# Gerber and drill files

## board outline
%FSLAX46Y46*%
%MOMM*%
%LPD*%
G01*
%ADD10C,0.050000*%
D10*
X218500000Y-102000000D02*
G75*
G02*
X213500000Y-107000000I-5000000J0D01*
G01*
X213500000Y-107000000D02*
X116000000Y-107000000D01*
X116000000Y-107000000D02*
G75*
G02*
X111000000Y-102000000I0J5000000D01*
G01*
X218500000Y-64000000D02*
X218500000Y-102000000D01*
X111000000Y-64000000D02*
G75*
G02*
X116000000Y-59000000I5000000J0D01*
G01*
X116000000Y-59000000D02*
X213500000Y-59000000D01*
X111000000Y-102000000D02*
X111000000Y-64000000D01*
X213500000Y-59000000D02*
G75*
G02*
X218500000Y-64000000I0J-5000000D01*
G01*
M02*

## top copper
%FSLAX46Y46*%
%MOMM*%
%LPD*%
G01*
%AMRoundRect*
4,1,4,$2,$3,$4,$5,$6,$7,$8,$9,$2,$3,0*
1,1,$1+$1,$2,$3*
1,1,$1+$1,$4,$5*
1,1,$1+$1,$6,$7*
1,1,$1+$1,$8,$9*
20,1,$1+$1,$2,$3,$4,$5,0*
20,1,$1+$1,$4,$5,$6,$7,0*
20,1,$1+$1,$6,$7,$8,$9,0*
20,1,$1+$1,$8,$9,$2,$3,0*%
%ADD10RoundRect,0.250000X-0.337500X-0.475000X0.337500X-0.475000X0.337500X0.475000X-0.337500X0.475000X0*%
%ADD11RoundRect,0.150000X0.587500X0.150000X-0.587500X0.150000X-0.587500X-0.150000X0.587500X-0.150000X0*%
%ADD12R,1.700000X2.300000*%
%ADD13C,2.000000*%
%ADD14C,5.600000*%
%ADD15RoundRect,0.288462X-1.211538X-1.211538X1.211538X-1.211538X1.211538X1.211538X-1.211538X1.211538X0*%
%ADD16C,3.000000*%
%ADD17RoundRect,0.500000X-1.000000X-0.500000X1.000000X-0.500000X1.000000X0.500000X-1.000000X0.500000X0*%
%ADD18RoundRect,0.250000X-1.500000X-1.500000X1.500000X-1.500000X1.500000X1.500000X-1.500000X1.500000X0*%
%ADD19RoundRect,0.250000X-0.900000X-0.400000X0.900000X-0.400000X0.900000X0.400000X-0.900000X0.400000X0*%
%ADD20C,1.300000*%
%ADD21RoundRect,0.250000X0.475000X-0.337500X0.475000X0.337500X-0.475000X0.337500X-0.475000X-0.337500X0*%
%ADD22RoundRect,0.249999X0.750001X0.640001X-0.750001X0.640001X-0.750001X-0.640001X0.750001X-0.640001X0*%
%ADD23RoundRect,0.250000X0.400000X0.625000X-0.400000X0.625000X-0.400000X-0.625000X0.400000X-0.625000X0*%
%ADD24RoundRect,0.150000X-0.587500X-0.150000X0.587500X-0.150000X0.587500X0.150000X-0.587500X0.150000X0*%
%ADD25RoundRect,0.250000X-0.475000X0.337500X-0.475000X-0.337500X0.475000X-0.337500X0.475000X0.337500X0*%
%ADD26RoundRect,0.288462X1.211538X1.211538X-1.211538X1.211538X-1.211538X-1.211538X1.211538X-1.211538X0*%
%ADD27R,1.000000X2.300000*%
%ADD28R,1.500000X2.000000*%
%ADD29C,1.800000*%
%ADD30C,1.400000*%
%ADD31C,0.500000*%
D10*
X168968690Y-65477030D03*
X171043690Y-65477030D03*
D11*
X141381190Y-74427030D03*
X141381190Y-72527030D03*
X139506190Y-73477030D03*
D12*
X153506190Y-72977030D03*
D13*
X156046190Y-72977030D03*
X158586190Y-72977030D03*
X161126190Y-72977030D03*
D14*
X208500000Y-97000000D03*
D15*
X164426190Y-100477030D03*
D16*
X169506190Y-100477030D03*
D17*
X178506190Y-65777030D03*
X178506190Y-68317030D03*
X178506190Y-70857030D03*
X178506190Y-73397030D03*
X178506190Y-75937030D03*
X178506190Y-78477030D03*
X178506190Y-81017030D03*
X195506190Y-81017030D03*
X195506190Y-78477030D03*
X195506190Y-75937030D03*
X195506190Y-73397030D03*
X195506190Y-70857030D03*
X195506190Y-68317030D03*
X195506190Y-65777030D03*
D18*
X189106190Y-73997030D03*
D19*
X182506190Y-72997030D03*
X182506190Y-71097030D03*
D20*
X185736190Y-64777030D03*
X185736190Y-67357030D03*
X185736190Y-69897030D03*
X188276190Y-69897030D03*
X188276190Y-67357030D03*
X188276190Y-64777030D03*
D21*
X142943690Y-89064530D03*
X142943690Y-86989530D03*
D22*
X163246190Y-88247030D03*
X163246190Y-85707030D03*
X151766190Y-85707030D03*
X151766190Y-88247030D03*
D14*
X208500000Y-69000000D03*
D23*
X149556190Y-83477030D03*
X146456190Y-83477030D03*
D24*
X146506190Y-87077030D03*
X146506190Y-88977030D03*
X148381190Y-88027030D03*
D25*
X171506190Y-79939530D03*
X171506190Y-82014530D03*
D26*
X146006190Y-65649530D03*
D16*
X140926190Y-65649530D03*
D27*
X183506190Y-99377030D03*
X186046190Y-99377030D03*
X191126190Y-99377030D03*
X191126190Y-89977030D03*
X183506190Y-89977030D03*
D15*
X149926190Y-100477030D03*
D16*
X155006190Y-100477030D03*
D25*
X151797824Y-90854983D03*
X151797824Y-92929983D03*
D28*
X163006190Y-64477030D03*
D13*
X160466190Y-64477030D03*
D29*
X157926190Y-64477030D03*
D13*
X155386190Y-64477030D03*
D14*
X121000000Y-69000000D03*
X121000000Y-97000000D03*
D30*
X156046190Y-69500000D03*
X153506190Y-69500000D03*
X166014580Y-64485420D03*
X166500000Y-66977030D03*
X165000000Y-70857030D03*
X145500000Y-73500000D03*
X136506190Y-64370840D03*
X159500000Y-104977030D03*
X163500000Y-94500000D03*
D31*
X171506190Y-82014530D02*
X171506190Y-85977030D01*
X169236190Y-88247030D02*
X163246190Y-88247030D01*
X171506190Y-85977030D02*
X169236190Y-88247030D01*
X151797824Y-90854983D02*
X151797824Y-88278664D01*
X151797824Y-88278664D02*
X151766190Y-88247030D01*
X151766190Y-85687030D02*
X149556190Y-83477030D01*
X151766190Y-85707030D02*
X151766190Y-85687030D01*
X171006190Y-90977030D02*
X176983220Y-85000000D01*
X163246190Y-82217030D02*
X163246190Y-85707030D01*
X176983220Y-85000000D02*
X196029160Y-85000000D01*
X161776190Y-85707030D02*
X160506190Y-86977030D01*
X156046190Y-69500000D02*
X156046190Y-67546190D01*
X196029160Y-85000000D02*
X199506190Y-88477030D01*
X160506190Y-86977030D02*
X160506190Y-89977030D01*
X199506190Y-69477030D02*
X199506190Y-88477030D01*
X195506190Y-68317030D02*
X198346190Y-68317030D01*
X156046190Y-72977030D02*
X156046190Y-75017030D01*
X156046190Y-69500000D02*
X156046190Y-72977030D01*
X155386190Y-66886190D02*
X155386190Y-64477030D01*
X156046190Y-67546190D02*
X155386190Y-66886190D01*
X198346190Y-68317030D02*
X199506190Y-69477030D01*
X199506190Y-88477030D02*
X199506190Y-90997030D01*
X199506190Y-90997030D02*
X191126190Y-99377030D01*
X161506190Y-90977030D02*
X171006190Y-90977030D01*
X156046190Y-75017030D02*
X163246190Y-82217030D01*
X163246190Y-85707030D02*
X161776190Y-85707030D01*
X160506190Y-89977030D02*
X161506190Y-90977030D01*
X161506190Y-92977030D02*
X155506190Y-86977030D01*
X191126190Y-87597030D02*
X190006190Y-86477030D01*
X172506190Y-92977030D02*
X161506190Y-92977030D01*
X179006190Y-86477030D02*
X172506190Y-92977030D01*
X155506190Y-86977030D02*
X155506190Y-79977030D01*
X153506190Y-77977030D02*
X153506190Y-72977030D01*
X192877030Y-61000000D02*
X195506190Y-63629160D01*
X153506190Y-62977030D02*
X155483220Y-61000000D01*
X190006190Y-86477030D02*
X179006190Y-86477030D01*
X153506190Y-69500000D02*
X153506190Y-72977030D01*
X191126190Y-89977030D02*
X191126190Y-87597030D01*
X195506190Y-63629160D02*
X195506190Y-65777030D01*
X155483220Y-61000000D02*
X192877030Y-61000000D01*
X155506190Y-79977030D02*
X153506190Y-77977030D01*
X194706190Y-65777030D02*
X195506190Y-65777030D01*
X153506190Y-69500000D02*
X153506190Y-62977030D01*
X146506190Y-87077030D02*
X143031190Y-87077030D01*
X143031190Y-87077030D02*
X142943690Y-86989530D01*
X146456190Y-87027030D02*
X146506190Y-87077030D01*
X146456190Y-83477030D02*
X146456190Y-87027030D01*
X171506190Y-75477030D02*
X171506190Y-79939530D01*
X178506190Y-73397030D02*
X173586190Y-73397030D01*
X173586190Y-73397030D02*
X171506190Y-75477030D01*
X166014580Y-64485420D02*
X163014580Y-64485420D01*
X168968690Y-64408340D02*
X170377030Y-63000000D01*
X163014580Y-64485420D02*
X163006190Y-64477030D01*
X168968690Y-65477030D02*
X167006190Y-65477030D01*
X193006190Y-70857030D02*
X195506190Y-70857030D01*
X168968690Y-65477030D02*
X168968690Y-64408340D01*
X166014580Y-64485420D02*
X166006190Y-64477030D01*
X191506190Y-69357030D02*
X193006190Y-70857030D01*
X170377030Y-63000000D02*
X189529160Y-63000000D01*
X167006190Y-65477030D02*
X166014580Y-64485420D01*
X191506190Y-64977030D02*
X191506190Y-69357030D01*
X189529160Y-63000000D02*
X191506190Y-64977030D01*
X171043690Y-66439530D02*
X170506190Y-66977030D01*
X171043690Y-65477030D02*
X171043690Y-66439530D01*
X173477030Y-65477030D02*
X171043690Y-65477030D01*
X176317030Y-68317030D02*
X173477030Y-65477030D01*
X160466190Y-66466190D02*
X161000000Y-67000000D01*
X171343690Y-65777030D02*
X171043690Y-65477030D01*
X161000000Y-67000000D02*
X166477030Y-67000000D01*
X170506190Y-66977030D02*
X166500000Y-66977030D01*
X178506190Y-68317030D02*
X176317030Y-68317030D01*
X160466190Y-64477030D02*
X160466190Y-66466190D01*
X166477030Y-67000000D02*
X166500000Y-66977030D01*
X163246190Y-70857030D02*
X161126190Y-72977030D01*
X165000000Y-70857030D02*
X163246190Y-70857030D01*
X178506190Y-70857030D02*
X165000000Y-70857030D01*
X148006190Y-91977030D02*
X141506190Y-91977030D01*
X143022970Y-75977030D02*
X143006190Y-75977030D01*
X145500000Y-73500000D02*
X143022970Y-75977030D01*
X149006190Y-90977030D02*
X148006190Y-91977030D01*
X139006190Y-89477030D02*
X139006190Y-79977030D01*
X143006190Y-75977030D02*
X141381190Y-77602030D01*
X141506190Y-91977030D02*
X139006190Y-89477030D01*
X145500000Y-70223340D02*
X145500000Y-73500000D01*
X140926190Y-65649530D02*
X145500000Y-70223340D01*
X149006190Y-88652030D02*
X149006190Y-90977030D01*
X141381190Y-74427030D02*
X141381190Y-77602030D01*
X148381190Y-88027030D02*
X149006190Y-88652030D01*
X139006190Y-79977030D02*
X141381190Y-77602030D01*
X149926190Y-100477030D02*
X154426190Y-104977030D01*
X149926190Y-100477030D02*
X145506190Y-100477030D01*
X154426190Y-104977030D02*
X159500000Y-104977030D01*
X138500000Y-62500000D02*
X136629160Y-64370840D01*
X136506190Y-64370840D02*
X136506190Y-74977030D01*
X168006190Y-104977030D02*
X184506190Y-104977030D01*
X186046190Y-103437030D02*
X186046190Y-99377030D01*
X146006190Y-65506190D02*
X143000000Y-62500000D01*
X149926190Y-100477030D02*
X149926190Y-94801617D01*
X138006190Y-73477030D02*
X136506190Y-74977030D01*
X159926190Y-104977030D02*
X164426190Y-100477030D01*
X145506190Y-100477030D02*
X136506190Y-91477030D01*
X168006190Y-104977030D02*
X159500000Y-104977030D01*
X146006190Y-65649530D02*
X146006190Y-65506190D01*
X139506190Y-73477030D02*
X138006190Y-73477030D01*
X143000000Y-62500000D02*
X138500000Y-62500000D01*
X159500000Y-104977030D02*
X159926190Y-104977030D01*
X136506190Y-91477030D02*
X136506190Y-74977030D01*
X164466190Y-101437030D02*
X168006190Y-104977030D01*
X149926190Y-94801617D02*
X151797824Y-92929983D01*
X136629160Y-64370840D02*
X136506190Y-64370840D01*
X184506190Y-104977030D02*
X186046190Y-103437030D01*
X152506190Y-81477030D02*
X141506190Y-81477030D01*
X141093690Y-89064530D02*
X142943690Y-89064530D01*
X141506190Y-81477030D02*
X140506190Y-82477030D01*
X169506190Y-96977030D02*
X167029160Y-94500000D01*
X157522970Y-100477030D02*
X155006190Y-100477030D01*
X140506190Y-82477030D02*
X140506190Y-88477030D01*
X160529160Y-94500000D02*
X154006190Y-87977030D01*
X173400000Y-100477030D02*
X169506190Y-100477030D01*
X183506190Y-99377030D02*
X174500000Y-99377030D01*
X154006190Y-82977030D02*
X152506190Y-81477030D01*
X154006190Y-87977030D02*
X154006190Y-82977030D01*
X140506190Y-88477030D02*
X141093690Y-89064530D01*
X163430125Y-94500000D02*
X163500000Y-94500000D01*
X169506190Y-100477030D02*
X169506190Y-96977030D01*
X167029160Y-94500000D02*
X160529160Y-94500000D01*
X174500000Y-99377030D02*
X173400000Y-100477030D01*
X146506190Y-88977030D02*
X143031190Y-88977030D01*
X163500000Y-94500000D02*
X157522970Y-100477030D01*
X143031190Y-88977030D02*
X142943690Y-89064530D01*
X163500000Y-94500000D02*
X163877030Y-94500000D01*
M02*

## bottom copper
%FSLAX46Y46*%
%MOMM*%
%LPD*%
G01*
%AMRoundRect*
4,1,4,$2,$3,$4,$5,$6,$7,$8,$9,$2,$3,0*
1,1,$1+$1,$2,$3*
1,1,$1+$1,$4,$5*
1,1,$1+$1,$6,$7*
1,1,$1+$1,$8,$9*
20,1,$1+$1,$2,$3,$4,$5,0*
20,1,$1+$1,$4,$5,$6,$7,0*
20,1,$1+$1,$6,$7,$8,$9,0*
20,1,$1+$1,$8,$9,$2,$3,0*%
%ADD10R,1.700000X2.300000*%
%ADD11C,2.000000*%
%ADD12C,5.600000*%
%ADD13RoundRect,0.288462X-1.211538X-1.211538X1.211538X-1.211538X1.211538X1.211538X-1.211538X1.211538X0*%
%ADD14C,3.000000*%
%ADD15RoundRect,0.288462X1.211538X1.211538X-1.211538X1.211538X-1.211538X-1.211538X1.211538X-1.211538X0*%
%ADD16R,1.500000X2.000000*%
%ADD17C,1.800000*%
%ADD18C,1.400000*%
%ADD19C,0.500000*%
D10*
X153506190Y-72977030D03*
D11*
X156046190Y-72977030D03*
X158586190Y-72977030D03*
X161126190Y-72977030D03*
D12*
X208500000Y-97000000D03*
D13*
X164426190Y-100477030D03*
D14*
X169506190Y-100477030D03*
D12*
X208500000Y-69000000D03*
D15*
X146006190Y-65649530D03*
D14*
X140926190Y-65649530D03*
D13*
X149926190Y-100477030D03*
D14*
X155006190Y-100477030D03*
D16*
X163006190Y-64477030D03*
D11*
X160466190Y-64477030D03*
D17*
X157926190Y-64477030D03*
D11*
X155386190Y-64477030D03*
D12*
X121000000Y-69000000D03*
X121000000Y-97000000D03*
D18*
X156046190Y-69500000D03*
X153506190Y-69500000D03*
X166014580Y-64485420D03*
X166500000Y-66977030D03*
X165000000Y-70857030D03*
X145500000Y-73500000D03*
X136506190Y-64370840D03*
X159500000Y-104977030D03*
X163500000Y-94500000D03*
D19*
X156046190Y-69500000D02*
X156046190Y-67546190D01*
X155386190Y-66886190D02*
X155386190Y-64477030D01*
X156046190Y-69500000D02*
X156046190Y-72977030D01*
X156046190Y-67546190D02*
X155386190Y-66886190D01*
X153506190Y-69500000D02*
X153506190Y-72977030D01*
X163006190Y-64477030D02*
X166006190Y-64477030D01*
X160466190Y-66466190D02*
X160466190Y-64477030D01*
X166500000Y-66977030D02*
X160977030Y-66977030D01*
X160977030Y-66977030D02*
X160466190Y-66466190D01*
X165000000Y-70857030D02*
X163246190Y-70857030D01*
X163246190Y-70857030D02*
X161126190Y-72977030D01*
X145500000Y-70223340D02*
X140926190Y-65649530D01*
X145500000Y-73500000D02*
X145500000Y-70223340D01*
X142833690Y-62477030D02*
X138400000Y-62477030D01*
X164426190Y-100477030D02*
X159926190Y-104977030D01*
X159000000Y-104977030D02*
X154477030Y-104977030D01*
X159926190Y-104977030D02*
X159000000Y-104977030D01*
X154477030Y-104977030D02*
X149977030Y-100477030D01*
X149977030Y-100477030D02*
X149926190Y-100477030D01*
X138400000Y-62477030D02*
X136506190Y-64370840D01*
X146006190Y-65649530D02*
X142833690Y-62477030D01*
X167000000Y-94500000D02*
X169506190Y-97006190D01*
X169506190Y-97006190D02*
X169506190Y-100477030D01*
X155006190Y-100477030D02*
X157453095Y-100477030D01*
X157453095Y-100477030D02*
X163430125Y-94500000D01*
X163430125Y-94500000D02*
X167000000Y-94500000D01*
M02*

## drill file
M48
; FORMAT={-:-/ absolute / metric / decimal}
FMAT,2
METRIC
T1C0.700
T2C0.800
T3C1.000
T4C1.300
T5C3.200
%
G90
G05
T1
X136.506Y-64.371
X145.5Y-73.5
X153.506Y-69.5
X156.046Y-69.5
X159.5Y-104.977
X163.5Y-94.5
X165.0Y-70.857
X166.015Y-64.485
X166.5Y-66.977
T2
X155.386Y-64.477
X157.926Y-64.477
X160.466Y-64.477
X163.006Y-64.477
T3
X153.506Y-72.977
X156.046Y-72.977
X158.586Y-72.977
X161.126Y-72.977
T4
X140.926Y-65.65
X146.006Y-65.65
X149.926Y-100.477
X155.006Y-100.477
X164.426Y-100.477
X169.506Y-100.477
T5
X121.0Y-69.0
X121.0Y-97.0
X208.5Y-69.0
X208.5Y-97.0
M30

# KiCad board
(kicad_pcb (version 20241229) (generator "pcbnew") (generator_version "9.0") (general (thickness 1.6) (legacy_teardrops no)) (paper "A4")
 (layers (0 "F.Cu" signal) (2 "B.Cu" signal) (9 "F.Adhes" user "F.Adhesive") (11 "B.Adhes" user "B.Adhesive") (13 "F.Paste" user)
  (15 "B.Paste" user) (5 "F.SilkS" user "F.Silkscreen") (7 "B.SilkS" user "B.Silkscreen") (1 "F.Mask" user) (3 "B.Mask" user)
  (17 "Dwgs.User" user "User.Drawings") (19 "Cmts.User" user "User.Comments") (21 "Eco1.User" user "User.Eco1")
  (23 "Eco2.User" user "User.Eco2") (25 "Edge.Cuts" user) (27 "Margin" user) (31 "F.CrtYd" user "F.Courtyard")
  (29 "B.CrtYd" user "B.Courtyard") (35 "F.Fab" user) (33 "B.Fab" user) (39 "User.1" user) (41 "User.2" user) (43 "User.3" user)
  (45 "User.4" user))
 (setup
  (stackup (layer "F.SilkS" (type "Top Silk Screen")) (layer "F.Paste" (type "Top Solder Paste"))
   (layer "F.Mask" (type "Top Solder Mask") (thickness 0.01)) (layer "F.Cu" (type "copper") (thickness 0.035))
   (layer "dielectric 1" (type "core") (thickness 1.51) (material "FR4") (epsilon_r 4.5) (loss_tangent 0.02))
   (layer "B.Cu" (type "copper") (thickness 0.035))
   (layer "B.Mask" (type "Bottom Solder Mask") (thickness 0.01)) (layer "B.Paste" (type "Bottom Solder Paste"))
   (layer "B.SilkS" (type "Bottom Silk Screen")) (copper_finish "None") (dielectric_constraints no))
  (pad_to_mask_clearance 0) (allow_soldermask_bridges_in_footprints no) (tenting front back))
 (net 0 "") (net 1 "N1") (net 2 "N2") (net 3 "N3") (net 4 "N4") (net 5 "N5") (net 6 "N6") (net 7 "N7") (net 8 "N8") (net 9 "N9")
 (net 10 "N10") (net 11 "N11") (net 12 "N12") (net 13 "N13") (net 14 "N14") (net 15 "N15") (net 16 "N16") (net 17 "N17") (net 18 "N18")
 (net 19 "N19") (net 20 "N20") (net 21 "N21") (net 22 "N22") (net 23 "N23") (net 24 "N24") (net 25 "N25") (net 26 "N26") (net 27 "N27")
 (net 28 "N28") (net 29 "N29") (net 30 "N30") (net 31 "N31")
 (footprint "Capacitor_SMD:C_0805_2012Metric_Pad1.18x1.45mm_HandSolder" (layer "F.Cu") (at 170.00619 65.47703)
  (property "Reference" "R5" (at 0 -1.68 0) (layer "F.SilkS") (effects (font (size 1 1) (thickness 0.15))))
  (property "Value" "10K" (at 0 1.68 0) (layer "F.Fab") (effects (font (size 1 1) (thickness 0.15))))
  (pad "1" smd roundrect (at -1.0375 0) (size 1.175 1.45) (layers "F.Cu" "F.Mask" "F.Paste") (roundrect_rratio 0.212766) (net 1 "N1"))
  (pad "2" smd roundrect (at 1.0375 0) (size 1.175 1.45) (layers "F.Cu" "F.Mask" "F.Paste") (roundrect_rratio 0.212766) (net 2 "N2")))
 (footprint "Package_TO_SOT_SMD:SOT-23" (layer "F.Cu") (at 140.44369 73.47703 180)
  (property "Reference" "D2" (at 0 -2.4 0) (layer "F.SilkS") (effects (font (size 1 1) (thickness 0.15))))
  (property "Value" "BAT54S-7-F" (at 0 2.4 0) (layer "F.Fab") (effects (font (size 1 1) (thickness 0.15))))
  (pad "1" smd roundrect (at -0.9375 -0.95 180) (size 1.475 0.6) (layers "F.Cu" "F.Mask" "F.Paste") (roundrect_rratio 0.25) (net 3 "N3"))
  (pad "2" smd roundrect (at -0.9375 0.95 180) (size 1.475 0.6) (layers "F.Cu" "F.Mask" "F.Paste") (roundrect_rratio 0.25) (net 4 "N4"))
  (pad "3" smd roundrect (at 0.9375 0 180) (size 1.475 0.6) (layers "F.Cu" "F.Mask" "F.Paste") (roundrect_rratio 0.25) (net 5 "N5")))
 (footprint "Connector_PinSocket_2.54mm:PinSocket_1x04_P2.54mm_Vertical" (layer "F.Cu") (at 153.50619 72.97703 90)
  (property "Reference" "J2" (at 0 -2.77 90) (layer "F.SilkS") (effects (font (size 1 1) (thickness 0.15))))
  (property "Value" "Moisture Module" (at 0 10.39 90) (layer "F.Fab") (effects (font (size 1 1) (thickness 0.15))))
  (pad "1" thru_hole rect (at 0 0 90) (size 2.3 1.7) (drill 1) (layers "*.Cu" "*.Mask") (remove_unused_layers no) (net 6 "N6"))
  (pad "2" thru_hole circle (at 0 2.54 90) (size 2 2) (drill 1) (layers "*.Cu" "*.Mask") (remove_unused_layers no) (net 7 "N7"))
  (pad "3" thru_hole circle (at 0 5.08 90) (size 2 2) (drill 1) (layers "*.Cu" "*.Mask") (remove_unused_layers no) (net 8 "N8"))
  (pad "4" thru_hole circle (at 0 7.62 90) (size 2 2) (drill 1) (layers "*.Cu" "*.Mask") (remove_unused_layers no) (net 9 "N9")))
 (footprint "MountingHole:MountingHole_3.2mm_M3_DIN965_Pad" (layer "F.Cu") (at 208.5 97)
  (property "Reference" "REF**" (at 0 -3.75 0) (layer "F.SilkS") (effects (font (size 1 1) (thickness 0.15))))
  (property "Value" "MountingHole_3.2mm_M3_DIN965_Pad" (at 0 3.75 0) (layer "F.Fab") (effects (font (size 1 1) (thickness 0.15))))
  (pad "1" thru_hole circle (at 0 0) (size 5.6 5.6) (drill 3.2) (layers "*.Cu" "*.Mask") (remove_unused_layers no) (zone_connect 2)))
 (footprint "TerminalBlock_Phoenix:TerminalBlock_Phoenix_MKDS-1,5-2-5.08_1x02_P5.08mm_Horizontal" (layer "F.Cu") (at 164.42619 100.47703)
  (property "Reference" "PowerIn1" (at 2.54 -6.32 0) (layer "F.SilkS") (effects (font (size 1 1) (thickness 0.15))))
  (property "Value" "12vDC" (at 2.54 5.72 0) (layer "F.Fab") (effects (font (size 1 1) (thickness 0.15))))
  (pad "1" thru_hole roundrect (at 0 0) (size 3 3) (drill 1.3) (layers "*.Cu" "*.Mask") (remove_unused_layers no)
   (roundrect_rratio 0.096154) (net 5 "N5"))
  (pad "2" thru_hole circle (at 5.08 0) (size 3 3) (drill 1.3) (layers "*.Cu" "*.Mask") (remove_unused_layers no) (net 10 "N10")))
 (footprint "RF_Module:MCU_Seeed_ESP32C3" (layer "F.Cu") (at 187.00619 73.39703)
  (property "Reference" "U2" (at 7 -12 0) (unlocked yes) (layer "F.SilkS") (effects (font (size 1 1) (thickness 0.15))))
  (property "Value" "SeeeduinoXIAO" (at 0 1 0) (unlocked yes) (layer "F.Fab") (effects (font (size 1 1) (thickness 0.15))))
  (pad "" smd roundrect (at 1.1 -0.4) (size 1.5 1.5) (layers "F.Paste") (roundrect_rratio 0.1666666667))
  (pad "" smd roundrect (at 1.1 1.6) (size 1.5 1.5) (layers "F.Paste") (roundrect_rratio 0.1666666667))
  (pad "" smd roundrect (at 3.1 -0.4) (size 1.5 1.5) (layers "F.Paste") (roundrect_rratio 0.1666666667))
  (pad "" smd roundrect (at 3.1 1.6) (size 1.5 1.5) (layers "F.Paste") (roundrect_rratio 0.1666666667))
  (pad "1" smd roundrect (at -8.5 -7.62) (size 3 2) (layers "F.Cu" "F.Mask" "F.Paste") (roundrect_rratio 0.25) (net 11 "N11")
   (thermal_bridge_angle 45))
  (pad "2" smd roundrect (at -8.5 -5.08) (size 3 2) (layers "F.Cu" "F.Mask" "F.Paste") (roundrect_rratio 0.25) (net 2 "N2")
   (thermal_bridge_angle 45))
  (pad "3" smd roundrect (at -8.5 -2.54) (size 3 2) (layers "F.Cu" "F.Mask" "F.Paste") (roundrect_rratio 0.25) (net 9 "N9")
   (thermal_bridge_angle 45))
  (pad "4" smd roundrect (at -8.5 0) (size 3 2) (layers "F.Cu" "F.Mask" "F.Paste") (roundrect_rratio 0.25) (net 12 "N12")
   (thermal_bridge_angle 45))
  (pad "5" smd roundrect (at -8.5 2.54) (size 3 2) (layers "F.Cu" "F.Mask" "F.Paste") (roundrect_rratio 0.25) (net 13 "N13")
   (thermal_bridge_angle 45))
  (pad "6" smd roundrect (at -8.5 5.08) (size 3 2) (layers "F.Cu" "F.Mask" "F.Paste") (roundrect_rratio 0.25) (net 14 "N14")
   (thermal_bridge_angle 45))
  (pad "7" smd roundrect (at -8.5 7.62) (size 3 2) (layers "F.Cu" "F.Mask" "F.Paste") (roundrect_rratio 0.25) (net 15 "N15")
   (thermal_bridge_angle 45))
  (pad "8" smd roundrect (at 8.5 7.62) (size 3 2) (layers "F.Cu" "F.Mask" "F.Paste") (roundrect_rratio 0.25) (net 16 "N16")
   (thermal_bridge_angle 45))
  (pad "9" smd roundrect (at 8.5 5.08) (size 3 2) (layers "F.Cu" "F.Mask" "F.Paste") (roundrect_rratio 0.25) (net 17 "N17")
   (thermal_bridge_angle 45))
  (pad "10" smd roundrect (at 8.5 2.54) (size 3 2) (layers "F.Cu" "F.Mask" "F.Paste") (roundrect_rratio 0.25) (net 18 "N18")
   (thermal_bridge_angle 45))
  (pad "11" smd roundrect (at 8.5 0) (size 3 2) (layers "F.Cu" "F.Mask" "F.Paste") (roundrect_rratio 0.25) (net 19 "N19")
   (thermal_bridge_angle 45))
  (pad "12" smd roundrect (at 8.5 -2.54) (size 3 2) (layers "F.Cu" "F.Mask" "F.Paste") (roundrect_rratio 0.25) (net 1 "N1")
   (thermal_bridge_angle 45))
  (pad "13" smd roundrect (at 8.5 -5.08) (size 3 2) (layers "F.Cu" "F.Mask" "F.Paste") (roundrect_rratio 0.25) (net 7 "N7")
   (thermal_bridge_angle 45))
  (pad "14" smd roundrect (at 8.5 -7.62) (size 3 2) (layers "F.Cu" "F.Mask" "F.Paste") (roundrect_rratio 0.25) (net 6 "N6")
   (thermal_bridge_angle 45))
  (pad "15" smd roundrect (at 2.1 0.6) (size 3.5 3.5) (layers "F.Cu" "F.Mask") (roundrect_rratio 0.07142857143) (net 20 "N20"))
  (pad "16" smd roundrect (at -4.5 -0.4) (size 2.3 1.3) (layers "F.Cu" "F.Mask" "F.Paste") (roundrect_rratio 0.1923076923) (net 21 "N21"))
  (pad "17" smd roundrect (at -4.5 -2.3) (size 2.3 1.3) (layers "F.Cu" "F.Mask" "F.Paste") (roundrect_rratio 0.1923076923) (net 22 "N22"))
  (pad "18" smd circle (at -1.27 -8.62) (size 1.3 1.3) (layers "F.Cu" "F.Mask" "F.Paste") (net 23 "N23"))
  (pad "19" smd circle (at -1.27 -6.04) (size 1.3 1.3) (layers "F.Cu" "F.Mask" "F.Paste") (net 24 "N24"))
  (pad "20" smd circle (at -1.27 -3.5) (size 1.3 1.3) (layers "F.Cu" "F.Mask" "F.Paste") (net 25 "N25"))
  (pad "21" smd circle (at 1.27 -3.5) (size 1.3 1.3) (layers "F.Cu" "F.Mask" "F.Paste"))
  (pad "22" smd circle (at 1.27 -6.04) (size 1.3 1.3) (layers "F.Cu" "F.Mask" "F.Paste"))
  (pad "23" smd circle (at 1.27 -8.62) (size 1.3 1.3) (layers "F.Cu" "F.Mask" "F.Paste")))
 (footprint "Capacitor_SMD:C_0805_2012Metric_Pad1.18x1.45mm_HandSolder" (layer "F.Cu") (at 142.94369 88.02703 90)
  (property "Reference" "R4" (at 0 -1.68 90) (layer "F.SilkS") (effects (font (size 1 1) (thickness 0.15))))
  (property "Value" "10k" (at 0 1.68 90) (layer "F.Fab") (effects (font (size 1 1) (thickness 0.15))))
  (pad "1" smd roundrect (at -1.0375 0 90) (size 1.175 1.45) (layers "F.Cu" "F.Mask" "F.Paste") (roundrect_rratio 0.212766) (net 10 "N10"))
  (pad "2" smd roundrect (at 1.0375 0 90) (size 1.175 1.45) (layers "F.Cu" "F.Mask" "F.Paste") (roundrect_rratio 0.212766) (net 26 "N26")))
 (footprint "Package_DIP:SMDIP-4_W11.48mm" (layer "F.Cu") (at 157.50619 86.97703 180)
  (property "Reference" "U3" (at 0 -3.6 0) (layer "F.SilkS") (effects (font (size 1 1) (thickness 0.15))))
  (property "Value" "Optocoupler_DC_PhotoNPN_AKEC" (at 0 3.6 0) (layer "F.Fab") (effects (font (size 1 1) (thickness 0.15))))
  (pad "1" smd roundrect (at -5.74 -1.27 180) (size 2 1.78) (layers "F.Cu" "F.Mask" "F.Paste") (roundrect_rratio 0.140449) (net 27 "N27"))
  (pad "2" smd roundrect (at -5.74 1.27 180) (size 2 1.78) (layers "F.Cu" "F.Mask" "F.Paste") (roundrect_rratio 0.140449) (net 7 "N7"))
  (pad "3" smd roundrect (at 5.74 1.27 180) (size 2 1.78) (layers "F.Cu" "F.Mask" "F.Paste") (roundrect_rratio 0.140449) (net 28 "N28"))
  (pad "4" smd roundrect (at 5.74 -1.27 180) (size 2 1.78) (layers "F.Cu" "F.Mask" "F.Paste") (roundrect_rratio 0.140449) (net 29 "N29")))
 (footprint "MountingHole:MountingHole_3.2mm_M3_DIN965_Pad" (layer "F.Cu") (at 208.5 69)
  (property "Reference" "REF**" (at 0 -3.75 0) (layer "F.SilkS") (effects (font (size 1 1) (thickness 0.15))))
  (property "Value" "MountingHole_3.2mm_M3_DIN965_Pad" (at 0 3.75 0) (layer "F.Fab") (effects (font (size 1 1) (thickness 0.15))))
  (pad "1" thru_hole circle (at 0 0) (size 5.6 5.6) (drill 3.2) (layers "*.Cu" "*.Mask") (remove_unused_layers no) (zone_connect 2)))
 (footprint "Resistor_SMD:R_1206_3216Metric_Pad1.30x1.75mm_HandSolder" (layer "F.Cu") (at 148.00619 83.47703 180)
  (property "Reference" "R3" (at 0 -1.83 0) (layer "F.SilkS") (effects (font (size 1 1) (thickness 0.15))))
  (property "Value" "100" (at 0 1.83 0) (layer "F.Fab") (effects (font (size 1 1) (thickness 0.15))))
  (pad "1" smd roundrect (at -1.55 0 180) (size 1.3 1.75) (layers "F.Cu" "F.Mask" "F.Paste") (roundrect_rratio 0.192308) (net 28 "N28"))
  (pad "2" smd roundrect (at 1.55 0 180) (size 1.3 1.75) (layers "F.Cu" "F.Mask" "F.Paste") (roundrect_rratio 0.192308) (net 26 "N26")))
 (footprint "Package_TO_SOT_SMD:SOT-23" (layer "F.Cu") (at 147.44369 88.02703)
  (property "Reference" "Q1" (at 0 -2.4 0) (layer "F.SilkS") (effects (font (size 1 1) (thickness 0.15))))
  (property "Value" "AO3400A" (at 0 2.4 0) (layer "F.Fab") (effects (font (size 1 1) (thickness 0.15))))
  (pad "1" smd roundrect (at -0.9375 -0.95) (size 1.475 0.6) (layers "F.Cu" "F.Mask" "F.Paste") (roundrect_rratio 0.25) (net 26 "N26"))
  (pad "2" smd roundrect (at -0.9375 0.95) (size 1.475 0.6) (layers "F.Cu" "F.Mask" "F.Paste") (roundrect_rratio 0.25) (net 10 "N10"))
  (pad "3" smd roundrect (at 0.9375 0) (size 1.475 0.6) (layers "F.Cu" "F.Mask" "F.Paste") (roundrect_rratio 0.25) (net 3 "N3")))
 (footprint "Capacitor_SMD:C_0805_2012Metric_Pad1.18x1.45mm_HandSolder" (layer "F.Cu") (at 171.50619 80.97703 -90)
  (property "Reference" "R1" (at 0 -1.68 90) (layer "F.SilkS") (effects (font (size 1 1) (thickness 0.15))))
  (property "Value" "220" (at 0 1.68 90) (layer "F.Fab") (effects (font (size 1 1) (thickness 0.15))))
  (pad "1" smd roundrect (at -1.0375 0 270) (size 1.175 1.45) (layers "F.Cu" "F.Mask" "F.Paste") (roundrect_rratio 0.212766) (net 12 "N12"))
  (pad "2" smd roundrect (at 1.0375 0 270) (size 1.175 1.45) (layers "F.Cu" "F.Mask" "F.Paste") (roundrect_rratio 0.212766) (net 27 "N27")))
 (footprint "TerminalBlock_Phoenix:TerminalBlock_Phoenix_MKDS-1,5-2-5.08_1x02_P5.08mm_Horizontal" (layer "F.Cu") (at 146.00619 65.64953 180)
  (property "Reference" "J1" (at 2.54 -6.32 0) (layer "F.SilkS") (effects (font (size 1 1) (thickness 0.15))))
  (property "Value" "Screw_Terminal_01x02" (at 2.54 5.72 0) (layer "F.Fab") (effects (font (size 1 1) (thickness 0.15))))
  (pad "1" thru_hole roundrect (at 0 0 180) (size 3 3) (drill 1.3) (layers "*.Cu" "*.Mask") (remove_unused_layers no)
   (roundrect_rratio 0.096154) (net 5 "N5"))
  (pad "2" thru_hole circle (at 5.08 0 180) (size 3 3) (drill 1.3) (layers "*.Cu" "*.Mask") (remove_unused_layers no) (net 3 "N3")))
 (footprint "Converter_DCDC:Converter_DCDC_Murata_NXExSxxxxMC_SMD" (layer "F.Cu") (at 188.58619 94.67703 90)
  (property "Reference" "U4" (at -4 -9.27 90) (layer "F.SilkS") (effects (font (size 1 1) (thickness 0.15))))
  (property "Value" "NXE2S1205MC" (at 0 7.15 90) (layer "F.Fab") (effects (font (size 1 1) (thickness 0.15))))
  (pad "1" smd rect (at -4.7 -5.08 90) (size 2.3 1) (layers "F.Cu" "F.Mask" "F.Paste") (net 10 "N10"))
  (pad "3" smd rect (at -4.7 -2.54 90) (size 2.3 1) (layers "F.Cu" "F.Mask" "F.Paste") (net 5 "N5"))
  (pad "7" smd rect (at -4.7 2.54 90) (size 2.3 1) (layers "F.Cu" "F.Mask" "F.Paste") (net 7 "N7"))
  (pad "8" smd rect (at 4.7 2.54 90) (size 2.3 1) (layers "F.Cu" "F.Mask" "F.Paste") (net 6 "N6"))
  (pad "14" smd rect (at 4.7 -5.08 90) (size 2.3 1) (layers "F.Cu" "F.Mask" "F.Paste") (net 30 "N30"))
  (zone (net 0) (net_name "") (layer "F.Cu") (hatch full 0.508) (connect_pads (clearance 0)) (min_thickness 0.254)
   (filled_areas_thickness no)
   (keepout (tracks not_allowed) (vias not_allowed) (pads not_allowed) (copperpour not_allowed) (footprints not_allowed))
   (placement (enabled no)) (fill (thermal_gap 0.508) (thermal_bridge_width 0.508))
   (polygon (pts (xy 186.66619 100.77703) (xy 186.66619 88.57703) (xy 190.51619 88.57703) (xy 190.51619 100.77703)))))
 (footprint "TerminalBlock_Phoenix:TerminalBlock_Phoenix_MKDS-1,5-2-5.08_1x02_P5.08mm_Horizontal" (layer "F.Cu") (at 149.92619 100.47703)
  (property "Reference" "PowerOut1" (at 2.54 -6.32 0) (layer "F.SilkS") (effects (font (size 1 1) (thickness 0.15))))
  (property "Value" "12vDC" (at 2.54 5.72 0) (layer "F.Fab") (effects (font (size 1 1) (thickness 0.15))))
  (pad "1" thru_hole roundrect (at 0 0) (size 3 3) (drill 1.3) (layers "*.Cu" "*.Mask") (remove_unused_layers no)
   (roundrect_rratio 0.096154) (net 5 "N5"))
  (pad "2" thru_hole circle (at 5.08 0) (size 3 3) (drill 1.3) (layers "*.Cu" "*.Mask") (remove_unused_layers no) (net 10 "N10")))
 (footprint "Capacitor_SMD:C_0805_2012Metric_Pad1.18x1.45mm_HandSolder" (layer "F.Cu") (at 151.797824 91.892483 -90)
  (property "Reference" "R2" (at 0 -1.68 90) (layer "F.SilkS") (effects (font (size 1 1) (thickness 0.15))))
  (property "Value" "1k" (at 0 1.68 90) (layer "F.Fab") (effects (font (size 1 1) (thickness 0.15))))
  (pad "1" smd roundrect (at -1.0375 0 270) (size 1.175 1.45) (layers "F.Cu" "F.Mask" "F.Paste") (roundrect_rratio 0.212766) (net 29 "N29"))
  (pad "2" smd roundrect (at 1.0375 0 270) (size 1.175 1.45) (layers "F.Cu" "F.Mask" "F.Paste") (roundrect_rratio 0.212766) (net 5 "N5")))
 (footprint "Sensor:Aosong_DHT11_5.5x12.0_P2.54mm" (layer "F.Cu") (at 163.00619 64.47703 -90)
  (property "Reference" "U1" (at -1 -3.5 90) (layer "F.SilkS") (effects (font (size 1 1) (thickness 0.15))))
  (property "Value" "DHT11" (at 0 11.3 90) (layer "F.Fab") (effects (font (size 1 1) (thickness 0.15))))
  (pad "1" thru_hole rect (at 0 0 270) (size 2 1.5) (drill 0.8) (layers "*.Cu" "*.Mask") (remove_unused_layers no) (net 1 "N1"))
  (pad "2" thru_hole circle (at 0 2.54 270) (size 2 2) (drill 0.8) (layers "*.Cu" "*.Mask") (remove_unused_layers no) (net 2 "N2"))
  (pad "3" thru_hole circle (at 0 5.08 270) (size 1.8 1.8) (drill 0.8) (layers "*.Cu" "*.Mask") (remove_unused_layers no) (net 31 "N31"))
  (pad "4" thru_hole circle (at 0 7.62 270) (size 2 2) (drill 0.8) (layers "*.Cu" "*.Mask") (remove_unused_layers no) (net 7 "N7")))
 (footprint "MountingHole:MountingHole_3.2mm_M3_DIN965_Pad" (layer "F.Cu") (at 121 69)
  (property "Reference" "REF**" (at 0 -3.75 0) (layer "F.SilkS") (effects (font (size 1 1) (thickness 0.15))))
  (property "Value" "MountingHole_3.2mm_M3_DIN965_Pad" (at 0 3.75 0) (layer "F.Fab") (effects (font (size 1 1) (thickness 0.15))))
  (pad "1" thru_hole circle (at 0 0) (size 5.6 5.6) (drill 3.2) (layers "*.Cu" "*.Mask") (remove_unused_layers no) (zone_connect 2)))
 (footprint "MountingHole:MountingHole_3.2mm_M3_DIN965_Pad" (layer "F.Cu") (at 121 97)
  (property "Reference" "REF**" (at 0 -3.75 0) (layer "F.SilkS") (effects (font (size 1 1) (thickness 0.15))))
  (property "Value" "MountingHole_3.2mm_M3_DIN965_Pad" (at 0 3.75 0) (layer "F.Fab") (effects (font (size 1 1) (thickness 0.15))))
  (pad "1" thru_hole circle (at 0 0) (size 5.6 5.6) (drill 3.2) (layers "*.Cu" "*.Mask") (remove_unused_layers no) (zone_connect 2)))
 (gr_arc (start 218.5 102) (mid 217.035534 105.535534) (end 213.5 107) (stroke (width 0.05) (type default)) (layer "Edge.Cuts"))
 (gr_line (start 213.5 107) (end 116 107) (stroke (width 0.05) (type default)) (layer "Edge.Cuts"))
 (gr_arc (start 116 107) (mid 112.464466 105.535534) (end 111 102) (stroke (width 0.05) (type default)) (layer "Edge.Cuts"))
 (gr_line (start 218.5 64) (end 218.5 102) (stroke (width 0.05) (type default)) (layer "Edge.Cuts"))
 (gr_arc (start 111 64) (mid 112.464466 60.464466) (end 116 59) (stroke (width 0.05) (type default)) (layer "Edge.Cuts"))
 (gr_line (start 116 59) (end 213.5 59) (stroke (width 0.05) (type default)) (layer "Edge.Cuts"))
 (gr_line (start 111 102) (end 111 64) (stroke (width 0.05) (type default)) (layer "Edge.Cuts"))
 (gr_arc (start 213.5 59) (mid 217.035534 60.464466) (end 218.5 64) (stroke (width 0.05) (type default)) (layer "Edge.Cuts"))
 (segment (start 171.50619 82.01453) (end 171.50619 85.97703) (width 0.5) (layer "F.Cu") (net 27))
 (segment (start 169.23619 88.24703) (end 163.24619 88.24703) (width 0.5) (layer "F.Cu") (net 27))
 (segment (start 171.50619 85.97703) (end 169.23619 88.24703) (width 0.5) (layer "F.Cu") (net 27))
 (segment (start 151.797824 90.854983) (end 151.797824 88.278664) (width 0.5) (layer "F.Cu") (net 29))
 (segment (start 151.797824 88.278664) (end 151.76619 88.24703) (width 0.5) (layer "F.Cu") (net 29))
 (segment (start 151.76619 85.68703) (end 149.55619 83.47703) (width 0.5) (layer "F.Cu") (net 28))
 (segment (start 151.76619 85.70703) (end 151.76619 85.68703) (width 0.5) (layer "F.Cu") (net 28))
 (segment (start 171.00619 90.97703) (end 176.98322 85) (width 0.5) (layer "F.Cu") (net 7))
 (segment (start 163.24619 82.21703) (end 163.24619 85.70703) (width 0.5) (layer "F.Cu") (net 7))
 (segment (start 176.98322 85) (end 196.02916 85) (width 0.5) (layer "F.Cu") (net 7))
 (segment (start 161.77619 85.70703) (end 160.50619 86.97703) (width 0.5) (layer "F.Cu") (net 7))
 (segment (start 156.04619 69.5) (end 156.04619 67.54619) (width 0.5) (layer "F.Cu") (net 7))
 (segment (start 196.02916 85) (end 199.50619 88.47703) (width 0.5) (layer "F.Cu") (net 7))
 (segment (start 160.50619 86.97703) (end 160.50619 89.97703) (width 0.5) (layer "F.Cu") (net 7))
 (segment (start 199.50619 69.47703) (end 199.50619 88.47703) (width 0.5) (layer "F.Cu") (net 7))
 (segment (start 195.50619 68.31703) (end 198.34619 68.31703) (width 0.5) (layer "F.Cu") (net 7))
 (segment (start 156.04619 72.97703) (end 156.04619 75.01703) (width 0.5) (layer "F.Cu") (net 7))
 (segment (start 156.04619 69.5) (end 156.04619 72.97703) (width 0.5) (layer "F.Cu") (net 7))
 (segment (start 155.38619 66.88619) (end 155.38619 64.47703) (width 0.5) (layer "F.Cu") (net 7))
 (segment (start 156.04619 67.54619) (end 155.38619 66.88619) (width 0.5) (layer "F.Cu") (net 7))
 (segment (start 198.34619 68.31703) (end 199.50619 69.47703) (width 0.5) (layer "F.Cu") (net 7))
 (segment (start 199.50619 88.47703) (end 199.50619 90.99703) (width 0.5) (layer "F.Cu") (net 7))
 (segment (start 199.50619 90.99703) (end 191.12619 99.37703) (width 0.5) (layer "F.Cu") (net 7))
 (segment (start 161.50619 90.97703) (end 171.00619 90.97703) (width 0.5) (layer "F.Cu") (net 7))
 (segment (start 156.04619 75.01703) (end 163.24619 82.21703) (width 0.5) (layer "F.Cu") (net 7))
 (segment (start 163.24619 85.70703) (end 161.77619 85.70703) (width 0.5) (layer "F.Cu") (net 7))
 (segment (start 160.50619 89.97703) (end 161.50619 90.97703) (width 0.5) (layer "F.Cu") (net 7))
 (via (at 156.04619 69.5) (size 1.4) (drill 0.7) (layers "F.Cu" "B.Cu") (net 7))
 (segment (start 156.04619 69.5) (end 156.04619 67.54619) (width 0.5) (layer "B.Cu") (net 7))
 (segment (start 155.38619 66.88619) (end 155.38619 64.47703) (width 0.5) (layer "B.Cu") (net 7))
 (segment (start 156.04619 69.5) (end 156.04619 72.97703) (width 0.5) (layer "B.Cu") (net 7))
 (segment (start 156.04619 67.54619) (end 155.38619 66.88619) (width 0.5) (layer "B.Cu") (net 7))
 (segment (start 161.50619 92.97703) (end 155.50619 86.97703) (width 0.5) (layer "F.Cu") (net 6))
 (segment (start 191.12619 87.59703) (end 190.00619 86.47703) (width 0.5) (layer "F.Cu") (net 6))
 (segment (start 172.50619 92.97703) (end 161.50619 92.97703) (width 0.5) (layer "F.Cu") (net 6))
 (segment (start 179.00619 86.47703) (end 172.50619 92.97703) (width 0.5) (layer "F.Cu") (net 6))
 (segment (start 155.50619 86.97703) (end 155.50619 79.97703) (width 0.5) (layer "F.Cu") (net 6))
 (segment (start 153.50619 77.97703) (end 153.50619 72.97703) (width 0.5) (layer "F.Cu") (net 6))
 (segment (start 192.87703 61) (end 195.50619 63.62916) (width 0.5) (layer "F.Cu") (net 6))
 (segment (start 153.50619 62.97703) (end 155.48322 61) (width 0.5) (layer "F.Cu") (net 6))
 (segment (start 190.00619 86.47703) (end 179.00619 86.47703) (width 0.5) (layer "F.Cu") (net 6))
 (segment (start 153.50619 69.5) (end 153.50619 72.97703) (width 0.5) (layer "F.Cu") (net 6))
 (segment (start 191.12619 89.97703) (end 191.12619 87.59703) (width 0.5) (layer "F.Cu") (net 6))
 (segment (start 195.50619 63.62916) (end 195.50619 65.77703) (width 0.5) (layer "F.Cu") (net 6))
 (segment (start 155.48322 61) (end 192.87703 61) (width 0.5) (layer "F.Cu") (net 6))
 (segment (start 155.50619 79.97703) (end 153.50619 77.97703) (width 0.5) (layer "F.Cu") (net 6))
 (segment (start 194.70619 65.77703) (end 195.50619 65.77703) (width 0.5) (layer "F.Cu") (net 6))
 (segment (start 153.50619 69.5) (end 153.50619 62.97703) (width 0.5) (layer "F.Cu") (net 6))
 (via (at 153.50619 69.5) (size 1.4) (drill 0.7) (layers "F.Cu" "B.Cu") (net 6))
 (segment (start 153.50619 69.5) (end 153.50619 72.97703) (width 0.5) (layer "B.Cu") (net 6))
 (segment (start 146.50619 87.07703) (end 143.03119 87.07703) (width 0.5) (layer "F.Cu") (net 26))
 (segment (start 143.03119 87.07703) (end 142.94369 86.98953) (width 0.5) (layer "F.Cu") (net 26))
 (segment (start 146.45619 87.02703) (end 146.50619 87.07703) (width 0.5) (layer "F.Cu") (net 26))
 (segment (start 146.45619 83.47703) (end 146.45619 87.02703) (width 0.5) (layer "F.Cu") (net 26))
 (segment (start 171.50619 75.47703) (end 171.50619 79.93953) (width 0.5) (layer "F.Cu") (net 12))
 (segment (start 178.50619 73.39703) (end 173.58619 73.39703) (width 0.5) (layer "F.Cu") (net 12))
 (segment (start 173.58619 73.39703) (end 171.50619 75.47703) (width 0.5) (layer "F.Cu") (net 12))
 (segment (start 166.01458 64.48542) (end 163.01458 64.48542) (width 0.5) (layer "F.Cu") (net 1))
 (segment (start 168.96869 64.40834) (end 170.37703 63) (width 0.5) (layer "F.Cu") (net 1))
 (segment (start 163.01458 64.48542) (end 163.00619 64.47703) (width 0.5) (layer "F.Cu") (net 1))
 (segment (start 168.96869 65.47703) (end 167.00619 65.47703) (width 0.5) (layer "F.Cu") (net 1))
 (segment (start 193.00619 70.85703) (end 195.50619 70.85703) (width 0.5) (layer "F.Cu") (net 1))
 (segment (start 168.96869 65.47703) (end 168.96869 64.40834) (width 0.5) (layer "F.Cu") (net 1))
 (segment (start 166.01458 64.48542) (end 166.00619 64.47703) (width 0.5) (layer "F.Cu") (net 1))
 (segment (start 191.50619 69.35703) (end 193.00619 70.85703) (width 0.5) (layer "F.Cu") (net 1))
 (segment (start 170.37703 63) (end 189.52916 63) (width 0.5) (layer "F.Cu") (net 1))
 (segment (start 167.00619 65.47703) (end 166.01458 64.48542) (width 0.5) (layer "F.Cu") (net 1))
 (segment (start 191.50619 64.97703) (end 191.50619 69.35703) (width 0.5) (layer "F.Cu") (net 1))
 (segment (start 189.52916 63) (end 191.50619 64.97703) (width 0.5) (layer "F.Cu") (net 1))
 (via (at 166.01458 64.48542) (size 1.4) (drill 0.7) (layers "F.Cu" "B.Cu") (free yes) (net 1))
 (segment (start 163.00619 64.47703) (end 166.00619 64.47703) (width 0.5) (layer "B.Cu") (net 1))
 (segment (start 171.04369 66.43953) (end 170.50619 66.97703) (width 0.5) (layer "F.Cu") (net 2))
 (segment (start 171.04369 65.47703) (end 171.04369 66.43953) (width 0.5) (layer "F.Cu") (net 2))
 (segment (start 173.47703 65.47703) (end 171.04369 65.47703) (width 0.5) (layer "F.Cu") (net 2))
 (segment (start 176.31703 68.31703) (end 173.47703 65.47703) (width 0.5) (layer "F.Cu") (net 2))
 (segment (start 160.46619 66.46619) (end 161 67) (width 0.5) (layer "F.Cu") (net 2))
 (segment (start 171.34369 65.77703) (end 171.04369 65.47703) (width 0.5) (layer "F.Cu") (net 2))
 (segment (start 161 67) (end 166.47703 67) (width 0.5) (layer "F.Cu") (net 2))
 (segment (start 170.50619 66.97703) (end 166.5 66.97703) (width 0.5) (layer "F.Cu") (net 2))
 (segment (start 178.50619 68.31703) (end 176.31703 68.31703) (width 0.5) (layer "F.Cu") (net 2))
 (segment (start 160.46619 64.47703) (end 160.46619 66.46619) (width 0.5) (layer "F.Cu") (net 2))
 (segment (start 166.47703 67) (end 166.5 66.97703) (width 0.5) (layer "F.Cu") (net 2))
 (via (at 166.5 66.97703) (size 1.4) (drill 0.7) (layers "F.Cu" "B.Cu") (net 2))
 (segment (start 160.46619 66.46619) (end 160.46619 64.47703) (width 0.5) (layer "B.Cu") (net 2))
 (segment (start 166.5 66.97703) (end 160.97703 66.97703) (width 0.5) (layer "B.Cu") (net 2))
 (segment (start 160.97703 66.97703) (end 160.46619 66.46619) (width 0.5) (layer "B.Cu") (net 2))
 (segment (start 163.24619 70.85703) (end 161.12619 72.97703) (width 0.5) (layer "F.Cu") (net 9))
 (segment (start 165 70.85703) (end 163.24619 70.85703) (width 0.5) (layer "F.Cu") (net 9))
 (segment (start 178.50619 70.85703) (end 165 70.85703) (width 0.5) (layer "F.Cu") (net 9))
 (via (at 165 70.85703) (size 1.4) (drill 0.7) (layers "F.Cu" "B.Cu") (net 9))
 (segment (start 165 70.85703) (end 163.24619 70.85703) (width 0.5) (layer "B.Cu") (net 9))
 (segment (start 163.24619 70.85703) (end 161.12619 72.97703) (width 0.5) (layer "B.Cu") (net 9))
 (segment (start 148.00619 91.97703) (end 141.50619 91.97703) (width 0.5) (layer "F.Cu") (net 3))
 (segment (start 143.02297 75.97703) (end 143.00619 75.97703) (width 0.5) (layer "F.Cu") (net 3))
 (segment (start 145.5 73.5) (end 143.02297 75.97703) (width 0.5) (layer "F.Cu") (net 3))
 (segment (start 149.00619 90.97703) (end 148.00619 91.97703) (width 0.5) (layer "F.Cu") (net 3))
 (segment (start 139.00619 89.47703) (end 139.00619 79.97703) (width 0.5) (layer "F.Cu") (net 3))
 (segment (start 143.00619 75.97703) (end 141.38119 77.60203) (width 0.5) (layer "F.Cu") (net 3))
 (segment (start 141.50619 91.97703) (end 139.00619 89.47703) (width 0.5) (layer "F.Cu") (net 3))
 (segment (start 145.5 70.22334) (end 145.5 73.5) (width 0.5) (layer "F.Cu") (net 3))
 (segment (start 140.92619 65.64953) (end 145.5 70.22334) (width 0.5) (layer "F.Cu") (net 3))
 (segment (start 149.00619 88.65203) (end 149.00619 90.97703) (width 0.5) (layer "F.Cu") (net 3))
 (segment (start 141.38119 74.42703) (end 141.38119 77.60203) (width 0.5) (layer "F.Cu") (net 3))
 (segment (start 148.38119 88.02703) (end 149.00619 88.65203) (width 0.5) (layer "F.Cu") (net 3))
 (segment (start 139.00619 79.97703) (end 141.38119 77.60203) (width 0.5) (layer "F.Cu") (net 3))
 (via (at 145.5 73.5) (size 1.4) (drill 0.7) (layers "F.Cu" "B.Cu") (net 3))
 (segment (start 145.5 70.22334) (end 140.92619 65.64953) (width 0.5) (layer "B.Cu") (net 3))
 (segment (start 145.5 73.5) (end 145.5 70.22334) (width 0.5) (layer "B.Cu") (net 3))
 (segment (start 149.92619 100.47703) (end 154.42619 104.97703) (width 0.5) (layer "F.Cu") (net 5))
 (segment (start 149.92619 100.47703) (end 145.50619 100.47703) (width 0.5) (layer "F.Cu") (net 5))
 (segment (start 154.42619 104.97703) (end 159.5 104.97703) (width 0.5) (layer "F.Cu") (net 5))
 (segment (start 138.5 62.5) (end 136.62916 64.37084) (width 0.5) (layer "F.Cu") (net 5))
 (segment (start 136.50619 64.37084) (end 136.50619 74.97703) (width 0.5) (layer "F.Cu") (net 5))
 (segment (start 168.00619 104.97703) (end 184.50619 104.97703) (width 0.5) (layer "F.Cu") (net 5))
 (segment (start 186.04619 103.43703) (end 186.04619 99.37703) (width 0.5) (layer "F.Cu") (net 5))
 (segment (start 146.00619 65.50619) (end 143 62.5) (width 0.5) (layer "F.Cu") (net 5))
 (segment (start 149.92619 100.47703) (end 149.92619 94.801617) (width 0.5) (layer "F.Cu") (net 5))
 (segment (start 138.00619 73.47703) (end 136.50619 74.97703) (width 0.5) (layer "F.Cu") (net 5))
 (segment (start 159.92619 104.97703) (end 164.42619 100.47703) (width 0.5) (layer "F.Cu") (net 5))
 (segment (start 145.50619 100.47703) (end 136.50619 91.47703) (width 0.5) (layer "F.Cu") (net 5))
 (segment (start 168.00619 104.97703) (end 159.5 104.97703) (width 0.5) (layer "F.Cu") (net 5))
 (segment (start 146.00619 65.64953) (end 146.00619 65.50619) (width 0.5) (layer "F.Cu") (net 5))
 (segment (start 139.50619 73.47703) (end 138.00619 73.47703) (width 0.5) (layer "F.Cu") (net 5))
 (segment (start 143 62.5) (end 138.5 62.5) (width 0.5) (layer "F.Cu") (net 5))
 (segment (start 159.5 104.97703) (end 159.92619 104.97703) (width 0.5) (layer "F.Cu") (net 5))
 (segment (start 136.50619 91.47703) (end 136.50619 74.97703) (width 0.5) (layer "F.Cu") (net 5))
 (segment (start 164.46619 101.43703) (end 168.00619 104.97703) (width 0.5) (layer "F.Cu") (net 5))
 (segment (start 149.92619 94.801617) (end 151.797824 92.929983) (width 0.5) (layer "F.Cu") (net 5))
 (segment (start 136.62916 64.37084) (end 136.50619 64.37084) (width 0.5) (layer "F.Cu") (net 5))
 (segment (start 184.50619 104.97703) (end 186.04619 103.43703) (width 0.5) (layer "F.Cu") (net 5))
 (via (at 136.50619 64.37084) (size 1.4) (drill 0.7) (layers "F.Cu" "B.Cu") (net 5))
 (via (at 159.5 104.97703) (size 1.4) (drill 0.7) (layers "F.Cu" "B.Cu") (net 5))
 (segment (start 142.83369 62.47703) (end 138.4 62.47703) (width 0.5) (layer "B.Cu") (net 5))
 (segment (start 164.42619 100.47703) (end 159.92619 104.97703) (width 0.5) (layer "B.Cu") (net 5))
 (segment (start 159 104.97703) (end 154.47703 104.97703) (width 0.5) (layer "B.Cu") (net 5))
 (segment (start 159.92619 104.97703) (end 159 104.97703) (width 0.5) (layer "B.Cu") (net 5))
 (segment (start 154.47703 104.97703) (end 149.97703 100.47703) (width 0.5) (layer "B.Cu") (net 5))
 (segment (start 149.97703 100.47703) (end 149.92619 100.47703) (width 0.5) (layer "B.Cu") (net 5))
 (segment (start 138.4 62.47703) (end 136.50619 64.37084) (width 0.5) (layer "B.Cu") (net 5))
 (segment (start 146.00619 65.64953) (end 142.83369 62.47703) (width 0.5) (layer "B.Cu") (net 5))
 (segment (start 152.50619 81.47703) (end 141.50619 81.47703) (width 0.5) (layer "F.Cu") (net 10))
 (segment (start 141.09369 89.06453) (end 142.94369 89.06453) (width 0.5) (layer "F.Cu") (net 10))
 (segment (start 141.50619 81.47703) (end 140.50619 82.47703) (width 0.5) (layer "F.Cu") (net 10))
 (segment (start 169.50619 96.97703) (end 167.02916 94.5) (width 0.5) (layer "F.Cu") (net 10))
 (segment (start 157.52297 100.47703) (end 155.00619 100.47703) (width 0.5) (layer "F.Cu") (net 10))
 (segment (start 140.50619 82.47703) (end 140.50619 88.47703) (width 0.5) (layer "F.Cu") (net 10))
 (segment (start 160.52916 94.5) (end 154.00619 87.97703) (width 0.5) (layer "F.Cu") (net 10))
 (segment (start 173.4 100.47703) (end 169.50619 100.47703) (width 0.5) (layer "F.Cu") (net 10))
 (segment (start 183.50619 99.37703) (end 174.5 99.37703) (width 0.5) (layer "F.Cu") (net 10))
 (segment (start 154.00619 82.97703) (end 152.50619 81.47703) (width 0.5) (layer "F.Cu") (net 10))
 (segment (start 154.00619 87.97703) (end 154.00619 82.97703) (width 0.5) (layer "F.Cu") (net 10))
 (segment (start 140.50619 88.47703) (end 141.09369 89.06453) (width 0.5) (layer "F.Cu") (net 10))
 (segment (start 163.430125 94.5) (end 163.5 94.5) (width 0.5) (layer "F.Cu") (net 10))
 (segment (start 169.50619 100.47703) (end 169.50619 96.97703) (width 0.5) (layer "F.Cu") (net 10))
 (segment (start 167.02916 94.5) (end 160.52916 94.5) (width 0.5) (layer "F.Cu") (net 10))
 (segment (start 174.5 99.37703) (end 173.4 100.47703) (width 0.5) (layer "F.Cu") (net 10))
 (segment (start 146.50619 88.97703) (end 143.03119 88.97703) (width 0.5) (layer "F.Cu") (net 10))
 (segment (start 163.5 94.5) (end 157.52297 100.47703) (width 0.5) (layer "F.Cu") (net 10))
 (segment (start 143.03119 88.97703) (end 142.94369 89.06453) (width 0.5) (layer "F.Cu") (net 10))
 (segment (start 163.5 94.5) (end 163.87703 94.5) (width 0.5) (layer "F.Cu") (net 10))
 (via (at 163.5 94.5) (size 1.4) (drill 0.7) (layers "F.Cu" "B.Cu") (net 10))
 (segment (start 167 94.5) (end 169.50619 97.00619) (width 0.5) (layer "B.Cu") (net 10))
 (segment (start 169.50619 97.00619) (end 169.50619 100.47703) (width 0.5) (layer "B.Cu") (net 10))
 (segment (start 155.00619 100.47703) (end 157.453095 100.47703) (width 0.5) (layer "B.Cu") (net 10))
 (segment (start 157.453095 100.47703) (end 163.430125 94.5) (width 0.5) (layer "B.Cu") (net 10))
 (segment (start 163.430125 94.5) (end 167 94.5) (width 0.5) (layer "B.Cu") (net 10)))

